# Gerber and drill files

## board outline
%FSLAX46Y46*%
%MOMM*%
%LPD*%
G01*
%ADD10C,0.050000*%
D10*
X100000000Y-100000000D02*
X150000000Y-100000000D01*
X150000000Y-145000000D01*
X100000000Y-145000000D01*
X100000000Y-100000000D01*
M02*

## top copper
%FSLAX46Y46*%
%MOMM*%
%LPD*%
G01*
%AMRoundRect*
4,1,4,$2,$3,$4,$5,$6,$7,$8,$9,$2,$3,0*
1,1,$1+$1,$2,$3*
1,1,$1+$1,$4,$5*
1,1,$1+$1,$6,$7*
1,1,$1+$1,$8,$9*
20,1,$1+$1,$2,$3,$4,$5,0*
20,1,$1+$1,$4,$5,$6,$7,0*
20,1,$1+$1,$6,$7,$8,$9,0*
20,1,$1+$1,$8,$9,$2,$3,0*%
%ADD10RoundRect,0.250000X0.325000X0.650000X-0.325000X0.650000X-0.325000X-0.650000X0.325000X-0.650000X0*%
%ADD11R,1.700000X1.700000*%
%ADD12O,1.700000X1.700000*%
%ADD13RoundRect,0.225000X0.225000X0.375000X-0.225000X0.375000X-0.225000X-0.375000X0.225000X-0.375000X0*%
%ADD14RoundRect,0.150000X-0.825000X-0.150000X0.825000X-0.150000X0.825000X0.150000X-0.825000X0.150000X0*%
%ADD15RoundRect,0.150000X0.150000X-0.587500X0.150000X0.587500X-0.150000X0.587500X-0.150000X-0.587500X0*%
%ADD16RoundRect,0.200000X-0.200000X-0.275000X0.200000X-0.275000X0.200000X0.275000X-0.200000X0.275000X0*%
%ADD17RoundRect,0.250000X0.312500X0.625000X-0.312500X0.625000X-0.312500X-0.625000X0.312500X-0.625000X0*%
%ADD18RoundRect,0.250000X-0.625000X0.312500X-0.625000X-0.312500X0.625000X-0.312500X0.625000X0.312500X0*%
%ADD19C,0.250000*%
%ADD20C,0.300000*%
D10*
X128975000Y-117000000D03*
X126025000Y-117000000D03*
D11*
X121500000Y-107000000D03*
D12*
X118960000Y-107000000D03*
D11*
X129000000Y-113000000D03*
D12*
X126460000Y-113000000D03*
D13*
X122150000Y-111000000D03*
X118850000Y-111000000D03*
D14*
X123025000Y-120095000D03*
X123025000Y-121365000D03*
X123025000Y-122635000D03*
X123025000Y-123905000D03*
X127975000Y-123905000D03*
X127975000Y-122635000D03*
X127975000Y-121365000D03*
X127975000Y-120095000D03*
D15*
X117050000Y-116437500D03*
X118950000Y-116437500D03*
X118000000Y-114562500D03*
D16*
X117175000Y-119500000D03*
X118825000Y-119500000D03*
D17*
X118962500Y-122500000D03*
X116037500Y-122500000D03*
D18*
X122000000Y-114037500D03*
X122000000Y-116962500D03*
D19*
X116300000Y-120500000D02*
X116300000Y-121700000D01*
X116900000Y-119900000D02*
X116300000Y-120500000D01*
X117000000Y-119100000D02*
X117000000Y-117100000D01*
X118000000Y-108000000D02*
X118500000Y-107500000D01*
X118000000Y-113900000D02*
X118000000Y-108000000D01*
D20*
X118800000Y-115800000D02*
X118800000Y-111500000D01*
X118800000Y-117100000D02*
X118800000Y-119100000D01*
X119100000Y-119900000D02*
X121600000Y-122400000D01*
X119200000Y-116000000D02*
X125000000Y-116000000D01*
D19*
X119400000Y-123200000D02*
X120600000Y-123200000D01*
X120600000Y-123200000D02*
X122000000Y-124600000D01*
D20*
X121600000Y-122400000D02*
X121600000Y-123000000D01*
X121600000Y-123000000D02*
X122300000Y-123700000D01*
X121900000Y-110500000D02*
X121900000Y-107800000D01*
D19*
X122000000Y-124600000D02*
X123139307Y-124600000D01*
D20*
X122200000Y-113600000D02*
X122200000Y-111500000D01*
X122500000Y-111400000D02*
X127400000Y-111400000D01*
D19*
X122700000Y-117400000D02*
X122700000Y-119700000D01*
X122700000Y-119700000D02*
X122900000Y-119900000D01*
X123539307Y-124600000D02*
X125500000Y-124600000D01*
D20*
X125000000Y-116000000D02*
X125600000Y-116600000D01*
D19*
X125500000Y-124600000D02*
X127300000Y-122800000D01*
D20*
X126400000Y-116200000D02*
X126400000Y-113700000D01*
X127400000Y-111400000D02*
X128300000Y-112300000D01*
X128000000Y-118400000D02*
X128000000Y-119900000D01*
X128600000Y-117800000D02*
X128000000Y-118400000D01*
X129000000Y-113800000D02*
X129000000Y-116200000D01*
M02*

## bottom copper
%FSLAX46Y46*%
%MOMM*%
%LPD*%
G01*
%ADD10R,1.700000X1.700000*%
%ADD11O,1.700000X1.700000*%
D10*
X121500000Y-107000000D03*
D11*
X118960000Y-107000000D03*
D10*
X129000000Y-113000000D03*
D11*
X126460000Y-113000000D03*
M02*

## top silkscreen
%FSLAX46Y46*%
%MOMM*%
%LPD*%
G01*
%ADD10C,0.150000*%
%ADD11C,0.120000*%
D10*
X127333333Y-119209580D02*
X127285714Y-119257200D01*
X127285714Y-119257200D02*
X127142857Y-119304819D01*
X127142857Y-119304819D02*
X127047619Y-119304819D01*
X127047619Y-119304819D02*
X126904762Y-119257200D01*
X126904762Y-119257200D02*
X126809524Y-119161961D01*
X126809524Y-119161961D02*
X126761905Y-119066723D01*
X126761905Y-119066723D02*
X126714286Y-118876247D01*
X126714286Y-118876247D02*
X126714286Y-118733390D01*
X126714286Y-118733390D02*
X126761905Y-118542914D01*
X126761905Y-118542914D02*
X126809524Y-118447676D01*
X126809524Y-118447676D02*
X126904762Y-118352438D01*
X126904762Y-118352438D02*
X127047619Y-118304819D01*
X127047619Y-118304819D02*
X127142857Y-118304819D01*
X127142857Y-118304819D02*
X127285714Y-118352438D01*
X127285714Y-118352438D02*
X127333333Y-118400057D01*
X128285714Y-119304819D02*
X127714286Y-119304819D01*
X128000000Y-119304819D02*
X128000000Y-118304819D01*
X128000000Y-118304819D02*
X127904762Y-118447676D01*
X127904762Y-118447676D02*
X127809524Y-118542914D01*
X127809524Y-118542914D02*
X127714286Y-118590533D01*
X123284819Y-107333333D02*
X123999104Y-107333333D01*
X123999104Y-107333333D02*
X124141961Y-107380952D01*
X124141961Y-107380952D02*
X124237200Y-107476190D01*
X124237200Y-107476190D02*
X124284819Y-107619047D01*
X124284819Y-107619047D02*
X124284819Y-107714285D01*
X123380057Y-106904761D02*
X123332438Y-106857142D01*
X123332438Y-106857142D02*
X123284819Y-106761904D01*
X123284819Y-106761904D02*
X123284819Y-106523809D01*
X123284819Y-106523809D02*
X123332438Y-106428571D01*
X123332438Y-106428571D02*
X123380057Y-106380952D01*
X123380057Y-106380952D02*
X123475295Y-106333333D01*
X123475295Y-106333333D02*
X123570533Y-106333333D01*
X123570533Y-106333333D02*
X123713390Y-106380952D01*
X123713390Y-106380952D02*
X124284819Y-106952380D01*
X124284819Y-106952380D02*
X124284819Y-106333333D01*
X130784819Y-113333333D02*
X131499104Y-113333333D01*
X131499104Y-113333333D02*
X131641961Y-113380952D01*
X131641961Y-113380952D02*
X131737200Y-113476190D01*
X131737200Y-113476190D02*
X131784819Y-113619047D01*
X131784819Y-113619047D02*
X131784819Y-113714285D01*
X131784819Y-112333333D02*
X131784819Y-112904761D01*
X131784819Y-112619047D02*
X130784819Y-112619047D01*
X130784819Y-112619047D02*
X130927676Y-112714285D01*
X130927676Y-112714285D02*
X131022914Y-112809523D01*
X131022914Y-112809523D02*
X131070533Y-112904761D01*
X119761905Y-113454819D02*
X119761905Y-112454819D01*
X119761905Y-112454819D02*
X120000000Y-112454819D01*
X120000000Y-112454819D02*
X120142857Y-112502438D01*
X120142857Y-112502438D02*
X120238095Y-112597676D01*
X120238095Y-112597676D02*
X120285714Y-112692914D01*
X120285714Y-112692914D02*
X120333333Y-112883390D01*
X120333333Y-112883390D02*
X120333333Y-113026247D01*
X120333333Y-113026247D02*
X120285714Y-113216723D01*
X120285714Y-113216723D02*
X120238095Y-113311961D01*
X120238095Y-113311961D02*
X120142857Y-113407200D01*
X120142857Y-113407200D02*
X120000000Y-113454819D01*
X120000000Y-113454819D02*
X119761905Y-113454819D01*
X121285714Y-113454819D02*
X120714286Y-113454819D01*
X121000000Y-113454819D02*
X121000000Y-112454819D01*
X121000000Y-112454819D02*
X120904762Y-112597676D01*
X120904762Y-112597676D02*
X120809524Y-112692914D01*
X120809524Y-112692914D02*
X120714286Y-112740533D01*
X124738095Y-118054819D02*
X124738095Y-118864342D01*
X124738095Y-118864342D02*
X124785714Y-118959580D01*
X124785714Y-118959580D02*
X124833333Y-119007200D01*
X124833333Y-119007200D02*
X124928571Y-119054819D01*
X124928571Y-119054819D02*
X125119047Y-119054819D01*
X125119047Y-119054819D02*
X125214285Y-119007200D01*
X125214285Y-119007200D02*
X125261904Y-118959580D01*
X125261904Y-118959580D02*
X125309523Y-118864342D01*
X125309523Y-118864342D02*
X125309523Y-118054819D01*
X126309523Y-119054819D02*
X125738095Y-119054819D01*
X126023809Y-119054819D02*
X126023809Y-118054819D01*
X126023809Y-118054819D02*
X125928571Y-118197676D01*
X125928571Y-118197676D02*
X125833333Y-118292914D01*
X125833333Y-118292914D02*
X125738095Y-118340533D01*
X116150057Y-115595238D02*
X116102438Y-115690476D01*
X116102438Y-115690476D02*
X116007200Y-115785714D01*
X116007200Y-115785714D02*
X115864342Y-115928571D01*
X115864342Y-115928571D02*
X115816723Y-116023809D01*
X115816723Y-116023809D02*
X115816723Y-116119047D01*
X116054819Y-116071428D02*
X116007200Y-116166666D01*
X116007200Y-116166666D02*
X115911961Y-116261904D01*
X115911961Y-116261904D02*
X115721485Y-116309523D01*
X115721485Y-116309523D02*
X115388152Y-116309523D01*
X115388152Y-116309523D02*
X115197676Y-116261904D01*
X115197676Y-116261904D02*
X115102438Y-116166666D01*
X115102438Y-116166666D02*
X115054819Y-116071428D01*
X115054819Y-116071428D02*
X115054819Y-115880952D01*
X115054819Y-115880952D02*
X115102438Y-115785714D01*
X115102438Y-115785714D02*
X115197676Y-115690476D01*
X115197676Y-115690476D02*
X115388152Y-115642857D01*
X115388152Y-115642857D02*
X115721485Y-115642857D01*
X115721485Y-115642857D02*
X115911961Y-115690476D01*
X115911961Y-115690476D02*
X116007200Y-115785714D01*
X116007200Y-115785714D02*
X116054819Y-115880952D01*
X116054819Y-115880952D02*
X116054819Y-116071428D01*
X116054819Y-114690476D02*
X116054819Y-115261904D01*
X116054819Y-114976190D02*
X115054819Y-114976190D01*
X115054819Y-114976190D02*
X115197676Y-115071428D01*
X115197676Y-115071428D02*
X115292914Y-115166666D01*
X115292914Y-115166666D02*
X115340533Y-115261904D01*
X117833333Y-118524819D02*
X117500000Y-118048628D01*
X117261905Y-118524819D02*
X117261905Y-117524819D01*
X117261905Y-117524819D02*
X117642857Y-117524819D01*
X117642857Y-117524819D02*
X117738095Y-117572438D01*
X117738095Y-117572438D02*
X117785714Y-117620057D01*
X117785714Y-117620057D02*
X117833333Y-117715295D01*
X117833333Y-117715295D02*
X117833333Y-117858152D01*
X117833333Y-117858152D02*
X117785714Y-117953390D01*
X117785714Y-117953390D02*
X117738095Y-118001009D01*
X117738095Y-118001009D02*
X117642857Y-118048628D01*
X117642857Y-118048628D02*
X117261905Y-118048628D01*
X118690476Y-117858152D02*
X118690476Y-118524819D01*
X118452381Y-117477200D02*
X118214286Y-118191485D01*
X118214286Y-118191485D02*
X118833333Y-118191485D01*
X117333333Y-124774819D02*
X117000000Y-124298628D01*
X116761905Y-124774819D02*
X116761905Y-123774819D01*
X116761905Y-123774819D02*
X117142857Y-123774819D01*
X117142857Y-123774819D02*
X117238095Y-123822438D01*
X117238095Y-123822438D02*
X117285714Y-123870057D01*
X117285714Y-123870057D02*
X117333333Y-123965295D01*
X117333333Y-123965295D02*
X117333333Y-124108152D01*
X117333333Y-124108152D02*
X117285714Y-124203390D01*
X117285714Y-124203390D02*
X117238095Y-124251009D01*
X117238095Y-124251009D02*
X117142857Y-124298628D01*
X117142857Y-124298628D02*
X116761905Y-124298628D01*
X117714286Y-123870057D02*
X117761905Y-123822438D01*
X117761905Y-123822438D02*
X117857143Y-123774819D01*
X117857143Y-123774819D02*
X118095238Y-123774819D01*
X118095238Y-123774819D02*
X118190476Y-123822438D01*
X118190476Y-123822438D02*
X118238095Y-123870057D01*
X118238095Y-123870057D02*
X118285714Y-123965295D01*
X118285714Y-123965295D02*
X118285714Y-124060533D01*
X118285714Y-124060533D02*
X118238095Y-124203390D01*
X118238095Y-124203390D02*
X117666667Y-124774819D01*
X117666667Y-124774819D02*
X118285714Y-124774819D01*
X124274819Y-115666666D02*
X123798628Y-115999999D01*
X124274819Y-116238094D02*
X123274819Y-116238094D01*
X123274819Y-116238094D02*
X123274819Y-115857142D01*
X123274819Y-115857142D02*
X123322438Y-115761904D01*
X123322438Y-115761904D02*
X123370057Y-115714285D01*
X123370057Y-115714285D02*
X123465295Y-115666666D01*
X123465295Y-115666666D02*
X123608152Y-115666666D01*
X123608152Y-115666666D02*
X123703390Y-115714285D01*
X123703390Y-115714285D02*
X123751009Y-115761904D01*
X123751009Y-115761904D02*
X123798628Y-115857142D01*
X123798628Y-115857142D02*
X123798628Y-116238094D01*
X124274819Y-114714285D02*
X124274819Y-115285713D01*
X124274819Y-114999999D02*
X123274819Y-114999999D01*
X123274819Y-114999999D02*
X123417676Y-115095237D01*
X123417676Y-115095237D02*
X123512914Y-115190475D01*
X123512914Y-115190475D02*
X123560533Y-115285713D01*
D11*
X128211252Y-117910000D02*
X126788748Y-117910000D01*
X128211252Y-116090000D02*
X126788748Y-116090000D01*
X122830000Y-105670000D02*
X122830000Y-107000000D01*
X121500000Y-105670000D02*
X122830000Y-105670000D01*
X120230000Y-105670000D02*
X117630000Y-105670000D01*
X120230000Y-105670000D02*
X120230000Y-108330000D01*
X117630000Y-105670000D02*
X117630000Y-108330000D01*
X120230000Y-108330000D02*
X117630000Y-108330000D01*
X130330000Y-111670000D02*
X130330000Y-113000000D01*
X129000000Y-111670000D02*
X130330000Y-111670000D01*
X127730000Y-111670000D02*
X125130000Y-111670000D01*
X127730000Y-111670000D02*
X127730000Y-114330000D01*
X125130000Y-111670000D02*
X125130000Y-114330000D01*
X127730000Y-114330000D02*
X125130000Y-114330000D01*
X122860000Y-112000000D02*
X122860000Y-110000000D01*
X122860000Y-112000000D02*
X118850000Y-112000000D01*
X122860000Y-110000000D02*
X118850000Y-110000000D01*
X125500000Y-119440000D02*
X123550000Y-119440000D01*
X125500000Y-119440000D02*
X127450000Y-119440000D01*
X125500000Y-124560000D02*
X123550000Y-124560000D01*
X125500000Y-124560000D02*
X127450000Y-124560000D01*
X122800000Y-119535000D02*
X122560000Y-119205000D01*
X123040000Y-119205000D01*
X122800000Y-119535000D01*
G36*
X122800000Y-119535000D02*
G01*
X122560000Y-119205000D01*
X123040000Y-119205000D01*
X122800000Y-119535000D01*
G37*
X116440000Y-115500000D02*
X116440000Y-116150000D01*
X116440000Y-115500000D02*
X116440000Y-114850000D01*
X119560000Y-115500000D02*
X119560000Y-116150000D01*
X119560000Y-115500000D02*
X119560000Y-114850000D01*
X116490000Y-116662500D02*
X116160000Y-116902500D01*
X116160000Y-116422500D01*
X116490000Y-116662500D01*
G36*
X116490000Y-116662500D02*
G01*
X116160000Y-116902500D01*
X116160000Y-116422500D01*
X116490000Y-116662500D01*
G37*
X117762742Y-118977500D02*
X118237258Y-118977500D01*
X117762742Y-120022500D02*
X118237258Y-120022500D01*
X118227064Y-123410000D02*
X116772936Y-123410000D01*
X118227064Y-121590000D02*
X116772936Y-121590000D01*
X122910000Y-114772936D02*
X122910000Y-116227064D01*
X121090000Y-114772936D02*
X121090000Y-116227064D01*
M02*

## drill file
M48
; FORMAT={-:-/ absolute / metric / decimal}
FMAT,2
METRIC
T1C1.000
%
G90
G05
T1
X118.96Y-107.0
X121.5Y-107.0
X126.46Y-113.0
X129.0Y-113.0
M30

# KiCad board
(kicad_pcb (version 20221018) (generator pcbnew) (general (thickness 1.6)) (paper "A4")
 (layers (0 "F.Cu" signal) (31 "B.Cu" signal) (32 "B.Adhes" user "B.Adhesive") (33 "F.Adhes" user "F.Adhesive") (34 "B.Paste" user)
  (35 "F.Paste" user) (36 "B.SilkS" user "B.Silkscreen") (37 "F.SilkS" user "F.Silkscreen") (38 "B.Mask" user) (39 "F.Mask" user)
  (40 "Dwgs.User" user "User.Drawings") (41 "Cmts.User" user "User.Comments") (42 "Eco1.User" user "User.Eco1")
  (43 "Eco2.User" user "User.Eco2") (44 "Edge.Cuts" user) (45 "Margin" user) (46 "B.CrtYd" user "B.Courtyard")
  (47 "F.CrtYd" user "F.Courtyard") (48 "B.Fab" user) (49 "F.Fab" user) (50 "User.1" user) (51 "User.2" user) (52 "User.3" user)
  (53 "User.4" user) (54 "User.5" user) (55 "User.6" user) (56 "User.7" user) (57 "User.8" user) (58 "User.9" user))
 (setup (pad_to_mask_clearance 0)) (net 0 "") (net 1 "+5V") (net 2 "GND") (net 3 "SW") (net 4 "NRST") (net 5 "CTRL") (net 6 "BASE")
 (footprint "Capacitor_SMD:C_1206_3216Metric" (layer "F.Cu") (at 127.5 117 180)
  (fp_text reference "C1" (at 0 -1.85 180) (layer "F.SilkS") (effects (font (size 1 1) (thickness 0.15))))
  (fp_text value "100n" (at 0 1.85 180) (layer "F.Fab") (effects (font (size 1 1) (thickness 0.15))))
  (fp_line (start -0.711252 -0.91) (end 0.711252 -0.91) (stroke (width 0.12) (type solid)) (layer "F.SilkS"))
  (fp_line (start -0.711252 0.91) (end 0.711252 0.91) (stroke (width 0.12) (type solid)) (layer "F.SilkS"))
  (pad "1" smd roundrect (at -1.475 0 180) (size 1.15 1.8) (layers "F.Cu" "F.Paste" "F.Mask") (roundrect_rratio 0.217391) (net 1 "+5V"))
  (pad "2" smd roundrect (at 1.475 0 180) (size 1.15 1.8) (layers "F.Cu" "F.Paste" "F.Mask") (roundrect_rratio 0.217391) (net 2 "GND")))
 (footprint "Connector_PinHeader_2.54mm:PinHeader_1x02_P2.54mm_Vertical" (layer "F.Cu") (at 121.5 107 -90)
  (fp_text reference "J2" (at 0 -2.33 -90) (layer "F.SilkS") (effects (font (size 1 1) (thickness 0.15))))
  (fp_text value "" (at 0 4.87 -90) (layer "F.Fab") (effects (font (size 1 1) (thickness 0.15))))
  (fp_line (start -1.33 -1.33) (end 0 -1.33) (stroke (width 0.12) (type solid)) (layer "F.SilkS"))
  (fp_line (start -1.33 0) (end -1.33 -1.33) (stroke (width 0.12) (type solid)) (layer "F.SilkS"))
  (fp_line (start -1.33 1.27) (end -1.33 3.87) (stroke (width 0.12) (type solid)) (layer "F.SilkS"))
  (fp_line (start -1.33 1.27) (end 1.33 1.27) (stroke (width 0.12) (type solid)) (layer "F.SilkS"))
  (fp_line (start -1.33 3.87) (end 1.33 3.87) (stroke (width 0.12) (type solid)) (layer "F.SilkS"))
  (fp_line (start 1.33 1.27) (end 1.33 3.87) (stroke (width 0.12) (type solid)) (layer "F.SilkS"))
  (pad "1" thru_hole rect (at 0 0 270) (size 1.7 1.7) (drill 1) (layers "*.Cu" "*.Mask") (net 1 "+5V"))
  (pad "2" thru_hole oval (at 0 2.54 270) (size 1.7 1.7) (drill 1) (layers "*.Cu" "*.Mask") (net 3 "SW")))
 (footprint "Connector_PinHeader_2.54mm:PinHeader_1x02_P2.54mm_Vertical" (layer "F.Cu") (at 129 113 -90)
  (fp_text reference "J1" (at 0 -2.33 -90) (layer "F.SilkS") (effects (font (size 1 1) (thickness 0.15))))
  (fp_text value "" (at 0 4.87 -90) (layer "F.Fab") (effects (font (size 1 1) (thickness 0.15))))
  (fp_line (start -1.33 -1.33) (end 0 -1.33) (stroke (width 0.12) (type solid)) (layer "F.SilkS"))
  (fp_line (start -1.33 0) (end -1.33 -1.33) (stroke (width 0.12) (type solid)) (layer "F.SilkS"))
  (fp_line (start -1.33 1.27) (end -1.33 3.87) (stroke (width 0.12) (type solid)) (layer "F.SilkS"))
  (fp_line (start -1.33 1.27) (end 1.33 1.27) (stroke (width 0.12) (type solid)) (layer "F.SilkS"))
  (fp_line (start -1.33 3.87) (end 1.33 3.87) (stroke (width 0.12) (type solid)) (layer "F.SilkS"))
  (fp_line (start 1.33 1.27) (end 1.33 3.87) (stroke (width 0.12) (type solid)) (layer "F.SilkS"))
  (pad "1" thru_hole rect (at 0 0 270) (size 1.7 1.7) (drill 1) (layers "*.Cu" "*.Mask") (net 1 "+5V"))
  (pad "2" thru_hole oval (at 0 2.54 270) (size 1.7 1.7) (drill 1) (layers "*.Cu" "*.Mask") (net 2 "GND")))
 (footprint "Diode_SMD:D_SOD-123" (layer "F.Cu") (at 120.5 111 180)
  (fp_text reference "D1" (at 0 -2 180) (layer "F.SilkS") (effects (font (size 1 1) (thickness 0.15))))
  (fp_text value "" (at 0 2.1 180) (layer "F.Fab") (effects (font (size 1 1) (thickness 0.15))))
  (fp_line (start -2.36 -1) (end -2.36 1) (stroke (width 0.12) (type solid)) (layer "F.SilkS"))
  (fp_line (start -2.36 -1) (end 1.65 -1) (stroke (width 0.12) (type solid)) (layer "F.SilkS"))
  (fp_line (start -2.36 1) (end 1.65 1) (stroke (width 0.12) (type solid)) (layer "F.SilkS"))
  (pad "1" smd roundrect (at -1.65 0 180) (size 0.9 1.2) (layers "F.Cu" "F.Paste" "F.Mask") (roundrect_rratio 0.25) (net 1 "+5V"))
  (pad "2" smd roundrect (at 1.65 0 180) (size 0.9 1.2) (layers "F.Cu" "F.Paste" "F.Mask") (roundrect_rratio 0.25) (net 2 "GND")))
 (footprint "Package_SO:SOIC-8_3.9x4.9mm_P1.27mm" (layer "F.Cu") (at 125.5 122)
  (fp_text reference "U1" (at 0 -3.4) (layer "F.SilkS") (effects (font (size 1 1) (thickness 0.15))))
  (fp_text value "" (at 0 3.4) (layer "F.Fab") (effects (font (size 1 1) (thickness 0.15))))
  (fp_line (start 0 -2.56) (end -1.95 -2.56) (stroke (width 0.12) (type solid)) (layer "F.SilkS"))
  (fp_line (start 0 -2.56) (end 1.95 -2.56) (stroke (width 0.12) (type solid)) (layer "F.SilkS"))
  (fp_line (start 0 2.56) (end -1.95 2.56) (stroke (width 0.12) (type solid)) (layer "F.SilkS"))
  (fp_line (start 0 2.56) (end 1.95 2.56) (stroke (width 0.12) (type solid)) (layer "F.SilkS"))
  (fp_poly
   (pts (xy -2.7 -2.465) (xy -2.94 -2.795) (xy -2.46 -2.795) (xy -2.7 -2.465)) (stroke (width 0.12) (type solid)) (fill solid)
   (layer "F.SilkS"))
  (pad "1" smd roundrect (at -2.475 -1.905) (size 1.95 0.6) (layers "F.Cu" "F.Paste" "F.Mask") (roundrect_rratio 0.25) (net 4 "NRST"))
  (pad "2" smd roundrect (at -2.475 -0.635) (size 1.95 0.6) (layers "F.Cu" "F.Paste" "F.Mask") (roundrect_rratio 0.25))
  (pad "3" smd roundrect (at -2.475 0.635) (size 1.95 0.6) (layers "F.Cu" "F.Paste" "F.Mask") (roundrect_rratio 0.25))
  (pad "4" smd roundrect (at -2.475 1.905) (size 1.95 0.6) (layers "F.Cu" "F.Paste" "F.Mask") (roundrect_rratio 0.25) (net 2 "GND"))
  (pad "5" smd roundrect (at 2.475 1.905) (size 1.95 0.6) (layers "F.Cu" "F.Paste" "F.Mask") (roundrect_rratio 0.25))
  (pad "6" smd roundrect (at 2.475 0.635) (size 1.95 0.6) (layers "F.Cu" "F.Paste" "F.Mask") (roundrect_rratio 0.25) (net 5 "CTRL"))
  (pad "7" smd roundrect (at 2.475 -0.635) (size 1.95 0.6) (layers "F.Cu" "F.Paste" "F.Mask") (roundrect_rratio 0.25))
  (pad "8" smd roundrect (at 2.475 -1.905) (size 1.95 0.6) (layers "F.Cu" "F.Paste" "F.Mask") (roundrect_rratio 0.25) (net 1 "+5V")))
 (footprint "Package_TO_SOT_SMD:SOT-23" (layer "F.Cu") (at 118 115.5 90)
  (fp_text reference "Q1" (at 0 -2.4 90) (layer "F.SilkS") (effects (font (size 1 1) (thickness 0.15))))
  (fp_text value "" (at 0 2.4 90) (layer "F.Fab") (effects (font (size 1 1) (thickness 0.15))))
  (fp_line (start 0 -1.56) (end -0.65 -1.56) (stroke (width 0.12) (type solid)) (layer "F.SilkS"))
  (fp_line (start 0 -1.56) (end 0.65 -1.56) (stroke (width 0.12) (type solid)) (layer "F.SilkS"))
  (fp_line (start 0 1.56) (end -0.65 1.56) (stroke (width 0.12) (type solid)) (layer "F.SilkS"))
  (fp_line (start 0 1.56) (end 0.65 1.56) (stroke (width 0.12) (type solid)) (layer "F.SilkS"))
  (fp_poly
   (pts (xy -1.1625 -1.51) (xy -1.4025 -1.84) (xy -0.9225 -1.84) (xy -1.1625 -1.51)) (stroke (width 0.12) (type solid)) (fill solid)
   (layer "F.SilkS"))
  (pad "1" smd roundrect (at -0.9375 -0.95 90) (size 1.475 0.6) (layers "F.Cu" "F.Paste" "F.Mask") (roundrect_rratio 0.25) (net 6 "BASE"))
  (pad "2" smd roundrect (at -0.9375 0.95 90) (size 1.475 0.6) (layers "F.Cu" "F.Paste" "F.Mask") (roundrect_rratio 0.25) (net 2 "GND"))
  (pad "3" smd roundrect (at 0.9375 0 90) (size 1.475 0.6) (layers "F.Cu" "F.Paste" "F.Mask") (roundrect_rratio 0.25) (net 3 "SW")))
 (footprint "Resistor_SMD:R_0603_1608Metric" (layer "F.Cu") (at 118 119.5)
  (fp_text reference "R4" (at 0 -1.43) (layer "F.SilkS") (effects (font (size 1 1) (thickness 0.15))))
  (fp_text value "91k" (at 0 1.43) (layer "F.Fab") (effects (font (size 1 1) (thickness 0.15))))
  (fp_line (start -0.237258 -0.5225) (end 0.237258 -0.5225) (stroke (width 0.12) (type solid)) (layer "F.SilkS"))
  (fp_line (start -0.237258 0.5225) (end 0.237258 0.5225) (stroke (width 0.12) (type solid)) (layer "F.SilkS"))
  (pad "1" smd roundrect (at -0.825 0) (size 0.8 0.95) (layers "F.Cu" "F.Paste" "F.Mask") (roundrect_rratio 0.25) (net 6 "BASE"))
  (pad "2" smd roundrect (at 0.825 0) (size 0.8 0.95) (layers "F.Cu" "F.Paste" "F.Mask") (roundrect_rratio 0.25) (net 2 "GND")))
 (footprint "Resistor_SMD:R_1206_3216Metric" (layer "F.Cu") (at 117.5 122.5 180)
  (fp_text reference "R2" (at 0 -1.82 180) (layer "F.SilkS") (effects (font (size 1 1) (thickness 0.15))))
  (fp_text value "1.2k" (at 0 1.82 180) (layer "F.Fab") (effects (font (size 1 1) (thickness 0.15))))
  (fp_line (start -0.727064 -0.91) (end 0.727064 -0.91) (stroke (width 0.12) (type solid)) (layer "F.SilkS"))
  (fp_line (start -0.727064 0.91) (end 0.727064 0.91) (stroke (width 0.12) (type solid)) (layer "F.SilkS"))
  (pad "1" smd roundrect (at -1.4625 0 180) (size 1.125 1.75) (layers "F.Cu" "F.Paste" "F.Mask") (roundrect_rratio 0.222222) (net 5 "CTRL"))
  (pad "2" smd roundrect (at 1.4625 0 180) (size 1.125 1.75) (layers "F.Cu" "F.Paste" "F.Mask") (roundrect_rratio 0.222222) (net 6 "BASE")))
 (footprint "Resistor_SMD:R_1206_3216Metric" (layer "F.Cu") (at 122 115.5 -90)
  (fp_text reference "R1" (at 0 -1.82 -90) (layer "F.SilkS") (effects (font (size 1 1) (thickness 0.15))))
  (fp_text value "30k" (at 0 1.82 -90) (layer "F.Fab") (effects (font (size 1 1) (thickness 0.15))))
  (fp_line (start -0.727064 -0.91) (end 0.727064 -0.91) (stroke (width 0.12) (type solid)) (layer "F.SilkS"))
  (fp_line (start -0.727064 0.91) (end 0.727064 0.91) (stroke (width 0.12) (type solid)) (layer "F.SilkS"))
  (pad "1" smd roundrect (at -1.4625 0 270) (size 1.125 1.75) (layers "F.Cu" "F.Paste" "F.Mask") (roundrect_rratio 0.222222) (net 1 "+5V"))
  (pad "2" smd roundrect (at 1.4625 0 270) (size 1.125 1.75) (layers "F.Cu" "F.Paste" "F.Mask") (roundrect_rratio 0.222222) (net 4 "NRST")))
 (gr_rect (start 100 100) (end 150 145) (stroke (width 0.05) (type default)) (fill none) (layer "Edge.Cuts"))
 (segment (start 116.3 120.5) (end 116.3 121.7) (width 0.25) (layer "F.Cu") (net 6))
 (segment (start 116.9 119.9) (end 116.3 120.5) (width 0.25) (layer "F.Cu") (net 6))
 (segment (start 117 119.1) (end 117 117.1) (width 0.25) (layer "F.Cu") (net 6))
 (segment (start 118 108) (end 118.5 107.5) (width 0.25) (layer "F.Cu") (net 3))
 (segment (start 118 113.9) (end 118 108) (width 0.25) (layer "F.Cu") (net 3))
 (segment (start 118.8 115.8) (end 118.8 111.5) (width 0.3) (layer "F.Cu") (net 2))
 (segment (start 118.8 117.1) (end 118.8 119.1) (width 0.3) (layer "F.Cu") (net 2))
 (segment (start 119.1 119.9) (end 121.6 122.4) (width 0.3) (layer "F.Cu") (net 2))
 (segment (start 119.2 116) (end 125 116) (width 0.3) (layer "F.Cu") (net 2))
 (segment (start 119.4 123.2) (end 120.6 123.2) (width 0.25) (layer "F.Cu") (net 5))
 (segment (start 120.6 123.2) (end 122 124.6) (width 0.25) (layer "F.Cu") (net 5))
 (segment (start 121.6 122.4) (end 121.6 123) (width 0.3) (layer "F.Cu") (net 2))
 (segment (start 121.6 123) (end 122.3 123.7) (width 0.3) (layer "F.Cu") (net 2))
 (segment (start 121.9 110.5) (end 121.9 107.8) (width 0.3) (layer "F.Cu") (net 1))
 (segment (start 122 124.6) (end 123.139307 124.6) (width 0.25) (layer "F.Cu") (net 5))
 (segment (start 122.2 113.6) (end 122.2 111.5) (width 0.3) (layer "F.Cu") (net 1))
 (segment (start 122.5 111.4) (end 127.4 111.4) (width 0.3) (layer "F.Cu") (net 1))
 (segment (start 122.7 117.4) (end 122.7 119.7) (width 0.25) (layer "F.Cu") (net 4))
 (segment (start 122.7 119.7) (end 122.9 119.9) (width 0.25) (layer "F.Cu") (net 4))
 (segment (start 123.539307 124.6) (end 125.5 124.6) (width 0.25) (layer "F.Cu") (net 5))
 (segment (start 125 116) (end 125.6 116.6) (width 0.3) (layer "F.Cu") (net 2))
 (segment (start 125.5 124.6) (end 127.3 122.8) (width 0.25) (layer "F.Cu") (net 5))
 (segment (start 126.4 116.2) (end 126.4 113.7) (width 0.3) (layer "F.Cu") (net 2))
 (segment (start 127.4 111.4) (end 128.3 112.3) (width 0.3) (layer "F.Cu") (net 1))
 (segment (start 128 118.4) (end 128 119.9) (width 0.3) (layer "F.Cu") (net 1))
 (segment (start 128.6 117.8) (end 128 118.4) (width 0.3) (layer "F.Cu") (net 1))
 (segment (start 129 113.8) (end 129 116.2) (width 0.3) (layer "F.Cu") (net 1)))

